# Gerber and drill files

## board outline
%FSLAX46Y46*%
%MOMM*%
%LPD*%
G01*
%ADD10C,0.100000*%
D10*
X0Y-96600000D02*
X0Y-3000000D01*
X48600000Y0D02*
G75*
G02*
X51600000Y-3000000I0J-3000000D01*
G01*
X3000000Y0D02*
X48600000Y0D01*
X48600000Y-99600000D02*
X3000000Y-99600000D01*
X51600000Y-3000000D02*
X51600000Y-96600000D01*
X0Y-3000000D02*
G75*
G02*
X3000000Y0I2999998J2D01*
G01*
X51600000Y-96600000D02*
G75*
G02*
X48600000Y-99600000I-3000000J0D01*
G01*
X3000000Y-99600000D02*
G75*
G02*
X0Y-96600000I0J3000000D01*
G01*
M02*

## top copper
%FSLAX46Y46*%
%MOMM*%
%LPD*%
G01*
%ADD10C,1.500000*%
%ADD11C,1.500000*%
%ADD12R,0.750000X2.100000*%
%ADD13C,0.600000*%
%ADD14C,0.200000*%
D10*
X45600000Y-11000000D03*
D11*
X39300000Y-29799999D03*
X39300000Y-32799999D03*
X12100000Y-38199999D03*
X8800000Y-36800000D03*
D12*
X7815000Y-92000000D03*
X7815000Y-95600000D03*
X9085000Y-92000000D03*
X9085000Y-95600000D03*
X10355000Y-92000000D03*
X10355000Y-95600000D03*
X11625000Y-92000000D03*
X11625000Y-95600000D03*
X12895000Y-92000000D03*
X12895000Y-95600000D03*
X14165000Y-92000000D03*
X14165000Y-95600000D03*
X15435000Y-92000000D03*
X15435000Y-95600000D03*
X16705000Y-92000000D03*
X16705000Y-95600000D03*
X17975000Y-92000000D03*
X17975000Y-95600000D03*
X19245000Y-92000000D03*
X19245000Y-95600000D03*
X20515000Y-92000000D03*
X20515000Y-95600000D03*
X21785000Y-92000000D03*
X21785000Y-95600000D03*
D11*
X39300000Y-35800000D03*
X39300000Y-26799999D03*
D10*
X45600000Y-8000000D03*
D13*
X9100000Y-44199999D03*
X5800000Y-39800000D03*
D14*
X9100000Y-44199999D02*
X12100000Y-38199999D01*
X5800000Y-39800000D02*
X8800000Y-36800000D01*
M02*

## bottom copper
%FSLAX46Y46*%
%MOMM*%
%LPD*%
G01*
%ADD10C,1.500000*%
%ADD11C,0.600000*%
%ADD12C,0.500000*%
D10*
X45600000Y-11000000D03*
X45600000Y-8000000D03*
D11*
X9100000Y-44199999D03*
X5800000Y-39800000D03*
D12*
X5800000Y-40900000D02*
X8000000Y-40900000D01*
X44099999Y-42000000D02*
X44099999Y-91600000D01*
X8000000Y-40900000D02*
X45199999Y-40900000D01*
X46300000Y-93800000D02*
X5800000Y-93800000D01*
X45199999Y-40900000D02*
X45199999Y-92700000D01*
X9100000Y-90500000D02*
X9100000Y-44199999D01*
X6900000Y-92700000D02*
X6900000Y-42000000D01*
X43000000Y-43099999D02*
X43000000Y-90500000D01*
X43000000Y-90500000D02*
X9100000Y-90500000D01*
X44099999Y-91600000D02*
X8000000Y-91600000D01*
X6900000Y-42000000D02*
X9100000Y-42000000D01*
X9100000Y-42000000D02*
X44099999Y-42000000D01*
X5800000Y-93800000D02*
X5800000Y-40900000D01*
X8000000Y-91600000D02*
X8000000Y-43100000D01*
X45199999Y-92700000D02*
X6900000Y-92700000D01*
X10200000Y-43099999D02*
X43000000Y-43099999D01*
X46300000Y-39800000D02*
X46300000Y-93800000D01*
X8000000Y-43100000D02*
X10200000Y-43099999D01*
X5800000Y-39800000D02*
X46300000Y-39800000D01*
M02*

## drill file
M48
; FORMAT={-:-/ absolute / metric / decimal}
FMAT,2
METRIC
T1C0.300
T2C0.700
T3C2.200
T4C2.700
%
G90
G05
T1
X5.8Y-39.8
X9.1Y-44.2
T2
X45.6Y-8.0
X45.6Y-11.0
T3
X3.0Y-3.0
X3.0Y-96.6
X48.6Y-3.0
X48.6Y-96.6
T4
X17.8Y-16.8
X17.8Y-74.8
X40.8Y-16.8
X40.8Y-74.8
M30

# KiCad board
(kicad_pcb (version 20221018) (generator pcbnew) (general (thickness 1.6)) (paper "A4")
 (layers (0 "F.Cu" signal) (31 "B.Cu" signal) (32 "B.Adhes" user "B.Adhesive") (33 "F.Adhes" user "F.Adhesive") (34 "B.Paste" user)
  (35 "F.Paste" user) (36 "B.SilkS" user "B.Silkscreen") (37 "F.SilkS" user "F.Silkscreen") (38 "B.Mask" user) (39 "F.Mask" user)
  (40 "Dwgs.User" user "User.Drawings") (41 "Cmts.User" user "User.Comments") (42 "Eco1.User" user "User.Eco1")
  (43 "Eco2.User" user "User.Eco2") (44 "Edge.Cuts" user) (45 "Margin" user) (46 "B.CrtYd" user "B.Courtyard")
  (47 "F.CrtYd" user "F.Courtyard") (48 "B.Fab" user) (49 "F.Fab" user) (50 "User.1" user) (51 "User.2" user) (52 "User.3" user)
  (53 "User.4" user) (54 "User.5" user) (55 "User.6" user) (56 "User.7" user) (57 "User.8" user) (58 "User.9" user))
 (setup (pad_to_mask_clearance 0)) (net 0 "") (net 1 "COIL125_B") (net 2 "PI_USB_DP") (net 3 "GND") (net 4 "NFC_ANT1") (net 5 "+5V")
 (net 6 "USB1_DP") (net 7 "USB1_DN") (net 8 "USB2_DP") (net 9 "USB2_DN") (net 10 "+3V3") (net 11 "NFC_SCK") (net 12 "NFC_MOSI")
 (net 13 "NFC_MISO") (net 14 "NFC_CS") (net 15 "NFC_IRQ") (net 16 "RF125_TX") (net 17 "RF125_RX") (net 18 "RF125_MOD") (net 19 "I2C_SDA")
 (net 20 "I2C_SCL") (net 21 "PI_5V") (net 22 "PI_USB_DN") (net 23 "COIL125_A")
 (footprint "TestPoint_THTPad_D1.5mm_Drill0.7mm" (layer "F.Cu") (at 45.6 11)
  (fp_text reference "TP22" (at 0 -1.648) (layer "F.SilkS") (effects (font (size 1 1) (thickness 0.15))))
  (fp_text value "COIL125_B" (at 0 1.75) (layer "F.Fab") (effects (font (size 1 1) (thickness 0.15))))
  (pad "1" thru_hole circle (at 0 0) (size 1.5 1.5) (drill 0.7) (layers "*.Cu" "*.Mask") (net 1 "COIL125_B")))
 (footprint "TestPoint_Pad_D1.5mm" (layer "F.Cu") (at 39.3 29.799999)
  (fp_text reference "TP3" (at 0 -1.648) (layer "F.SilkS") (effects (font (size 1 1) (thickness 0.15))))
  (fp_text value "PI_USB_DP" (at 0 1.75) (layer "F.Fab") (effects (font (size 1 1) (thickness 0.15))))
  (pad "1" smd circle (at 0 0) (size 1.5 1.5) (layers "F.Cu" "F.Mask") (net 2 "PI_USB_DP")))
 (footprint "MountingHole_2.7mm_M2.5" (layer "F.Cu") (at 17.8 16.799999)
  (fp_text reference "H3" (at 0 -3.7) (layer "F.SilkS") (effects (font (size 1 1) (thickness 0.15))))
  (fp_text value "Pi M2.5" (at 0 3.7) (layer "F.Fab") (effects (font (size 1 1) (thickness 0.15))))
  (pad "" np_thru_hole circle (at 0 0) (size 2.7 2.7) (drill 2.7) (layers "*.Cu" "*.Mask")))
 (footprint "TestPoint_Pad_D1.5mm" (layer "F.Cu") (at 39.3 32.799999)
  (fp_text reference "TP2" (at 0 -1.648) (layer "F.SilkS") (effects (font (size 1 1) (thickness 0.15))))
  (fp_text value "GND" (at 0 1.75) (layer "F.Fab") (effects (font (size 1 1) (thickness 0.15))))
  (pad "1" smd circle (at 0 0) (size 1.5 1.5) (layers "F.Cu" "F.Mask") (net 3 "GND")))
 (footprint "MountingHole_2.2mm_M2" (layer "F.Cu") (at 48.6 3)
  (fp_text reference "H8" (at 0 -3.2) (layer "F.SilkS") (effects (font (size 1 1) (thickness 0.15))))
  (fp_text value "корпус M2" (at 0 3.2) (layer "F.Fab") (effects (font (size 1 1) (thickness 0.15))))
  (pad "" np_thru_hole circle (at 0 0) (size 2.2 2.2) (drill 2.2) (layers "*.Cu" "*.Mask")))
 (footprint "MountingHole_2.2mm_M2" (layer "F.Cu") (at 3 3)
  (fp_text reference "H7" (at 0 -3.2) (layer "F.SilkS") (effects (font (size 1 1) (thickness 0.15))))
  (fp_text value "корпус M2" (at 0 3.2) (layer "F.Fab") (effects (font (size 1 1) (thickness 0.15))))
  (pad "" np_thru_hole circle (at 0 0) (size 2.2 2.2) (drill 2.2) (layers "*.Cu" "*.Mask")))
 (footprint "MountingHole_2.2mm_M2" (layer "F.Cu") (at 3 96.6)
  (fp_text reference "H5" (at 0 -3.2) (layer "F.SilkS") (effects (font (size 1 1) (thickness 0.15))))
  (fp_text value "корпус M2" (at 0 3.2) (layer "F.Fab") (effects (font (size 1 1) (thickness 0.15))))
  (pad "" np_thru_hole circle (at 0 0) (size 2.2 2.2) (drill 2.2) (layers "*.Cu" "*.Mask")))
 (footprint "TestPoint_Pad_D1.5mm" (layer "F.Cu") (at 12.1 38.199999)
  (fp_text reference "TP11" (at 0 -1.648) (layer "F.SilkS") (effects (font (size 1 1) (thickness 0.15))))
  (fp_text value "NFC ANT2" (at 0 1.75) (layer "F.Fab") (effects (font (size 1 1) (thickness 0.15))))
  (pad "1" smd circle (at 0 0) (size 1.5 1.5) (layers "F.Cu" "F.Mask") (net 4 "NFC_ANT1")))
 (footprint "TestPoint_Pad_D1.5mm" (layer "F.Cu") (at 8.8 36.8)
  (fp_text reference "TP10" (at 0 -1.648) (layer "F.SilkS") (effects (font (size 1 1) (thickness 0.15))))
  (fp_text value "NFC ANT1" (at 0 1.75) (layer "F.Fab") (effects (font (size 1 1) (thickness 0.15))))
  (pad "1" smd circle (at 0 0) (size 1.5 1.5) (layers "F.Cu" "F.Mask") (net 4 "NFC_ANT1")))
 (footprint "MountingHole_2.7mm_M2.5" (layer "F.Cu") (at 40.8 16.799999)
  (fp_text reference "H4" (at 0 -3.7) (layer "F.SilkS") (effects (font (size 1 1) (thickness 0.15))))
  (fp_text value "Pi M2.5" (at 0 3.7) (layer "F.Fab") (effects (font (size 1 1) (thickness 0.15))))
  (pad "" np_thru_hole circle (at 0 0) (size 2.7 2.7) (drill 2.7) (layers "*.Cu" "*.Mask")))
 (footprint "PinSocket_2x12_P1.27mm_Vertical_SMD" (layer "F.Cu") (at 14.8 93.8 90)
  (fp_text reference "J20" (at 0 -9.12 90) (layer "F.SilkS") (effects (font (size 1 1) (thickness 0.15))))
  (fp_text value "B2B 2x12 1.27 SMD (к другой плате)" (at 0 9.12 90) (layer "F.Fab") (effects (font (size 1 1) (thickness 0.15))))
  (pad "1" smd rect (at 1.8 -6.985 90) (size 2.1 0.75) (layers "F.Cu" "F.Paste" "F.Mask") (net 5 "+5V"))
  (pad "2" smd rect (at -1.8 -6.985 90) (size 2.1 0.75) (layers "F.Cu" "F.Paste" "F.Mask") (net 5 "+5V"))
  (pad "3" smd rect (at 1.8 -5.715 90) (size 2.1 0.75) (layers "F.Cu" "F.Paste" "F.Mask") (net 3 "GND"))
  (pad "4" smd rect (at -1.8 -5.715 90) (size 2.1 0.75) (layers "F.Cu" "F.Paste" "F.Mask") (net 3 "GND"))
  (pad "5" smd rect (at 1.8 -4.445 90) (size 2.1 0.75) (layers "F.Cu" "F.Paste" "F.Mask") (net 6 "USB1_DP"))
  (pad "6" smd rect (at -1.8 -4.445 90) (size 2.1 0.75) (layers "F.Cu" "F.Paste" "F.Mask") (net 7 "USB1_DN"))
  (pad "7" smd rect (at 1.8 -3.175 90) (size 2.1 0.75) (layers "F.Cu" "F.Paste" "F.Mask") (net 3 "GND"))
  (pad "8" smd rect (at -1.8 -3.175 90) (size 2.1 0.75) (layers "F.Cu" "F.Paste" "F.Mask") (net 3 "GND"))
  (pad "9" smd rect (at 1.8 -1.905 90) (size 2.1 0.75) (layers "F.Cu" "F.Paste" "F.Mask") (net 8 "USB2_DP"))
  (pad "10" smd rect (at -1.8 -1.905 90) (size 2.1 0.75) (layers "F.Cu" "F.Paste" "F.Mask") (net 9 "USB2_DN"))
  (pad "11" smd rect (at 1.8 -0.635 90) (size 2.1 0.75) (layers "F.Cu" "F.Paste" "F.Mask") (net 3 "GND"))
  (pad "12" smd rect (at -1.8 -0.635 90) (size 2.1 0.75) (layers "F.Cu" "F.Paste" "F.Mask") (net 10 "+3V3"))
  (pad "13" smd rect (at 1.8 0.635 90) (size 2.1 0.75) (layers "F.Cu" "F.Paste" "F.Mask") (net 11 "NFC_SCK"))
  (pad "14" smd rect (at -1.8 0.635 90) (size 2.1 0.75) (layers "F.Cu" "F.Paste" "F.Mask") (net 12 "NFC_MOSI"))
  (pad "15" smd rect (at 1.8 1.905 90) (size 2.1 0.75) (layers "F.Cu" "F.Paste" "F.Mask") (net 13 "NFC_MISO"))
  (pad "16" smd rect (at -1.8 1.905 90) (size 2.1 0.75) (layers "F.Cu" "F.Paste" "F.Mask") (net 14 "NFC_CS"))
  (pad "17" smd rect (at 1.8 3.175 90) (size 2.1 0.75) (layers "F.Cu" "F.Paste" "F.Mask") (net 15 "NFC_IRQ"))
  (pad "18" smd rect (at -1.8 3.175 90) (size 2.1 0.75) (layers "F.Cu" "F.Paste" "F.Mask") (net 3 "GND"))
  (pad "19" smd rect (at 1.8 4.445 90) (size 2.1 0.75) (layers "F.Cu" "F.Paste" "F.Mask") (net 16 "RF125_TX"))
  (pad "20" smd rect (at -1.8 4.445 90) (size 2.1 0.75) (layers "F.Cu" "F.Paste" "F.Mask") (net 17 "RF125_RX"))
  (pad "21" smd rect (at 1.8 5.715 90) (size 2.1 0.75) (layers "F.Cu" "F.Paste" "F.Mask") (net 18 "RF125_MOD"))
  (pad "22" smd rect (at -1.8 5.715 90) (size 2.1 0.75) (layers "F.Cu" "F.Paste" "F.Mask") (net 3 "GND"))
  (pad "23" smd rect (at 1.8 6.985 90) (size 2.1 0.75) (layers "F.Cu" "F.Paste" "F.Mask") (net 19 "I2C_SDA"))
  (pad "24" smd rect (at -1.8 6.985 90) (size 2.1 0.75) (layers "F.Cu" "F.Paste" "F.Mask") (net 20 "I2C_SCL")))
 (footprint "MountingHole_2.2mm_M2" (layer "F.Cu") (at 48.6 96.6)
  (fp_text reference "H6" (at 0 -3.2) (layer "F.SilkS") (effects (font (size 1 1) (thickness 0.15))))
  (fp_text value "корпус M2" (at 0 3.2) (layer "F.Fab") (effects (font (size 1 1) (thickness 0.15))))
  (pad "" np_thru_hole circle (at 0 0) (size 2.2 2.2) (drill 2.2) (layers "*.Cu" "*.Mask")))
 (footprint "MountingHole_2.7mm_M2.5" (layer "F.Cu") (at 40.8 74.8)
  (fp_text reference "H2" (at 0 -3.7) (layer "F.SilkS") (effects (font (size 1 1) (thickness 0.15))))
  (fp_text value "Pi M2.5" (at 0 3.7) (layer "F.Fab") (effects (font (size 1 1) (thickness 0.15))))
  (pad "" np_thru_hole circle (at 0 0) (size 2.7 2.7) (drill 2.7) (layers "*.Cu" "*.Mask")))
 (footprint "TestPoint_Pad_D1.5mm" (layer "F.Cu") (at 39.3 35.8)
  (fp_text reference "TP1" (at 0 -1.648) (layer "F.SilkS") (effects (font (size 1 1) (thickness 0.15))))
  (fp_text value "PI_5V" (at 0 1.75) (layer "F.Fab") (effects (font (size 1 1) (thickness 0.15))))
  (pad "1" smd circle (at 0 0) (size 1.5 1.5) (layers "F.Cu" "F.Mask") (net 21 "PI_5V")))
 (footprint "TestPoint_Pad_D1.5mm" (layer "F.Cu") (at 39.3 26.799999)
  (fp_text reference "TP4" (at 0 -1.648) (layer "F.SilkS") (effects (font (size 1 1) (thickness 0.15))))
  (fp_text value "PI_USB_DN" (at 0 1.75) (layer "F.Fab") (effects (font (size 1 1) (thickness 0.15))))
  (pad "1" smd circle (at 0 0) (size 1.5 1.5) (layers "F.Cu" "F.Mask") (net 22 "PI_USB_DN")))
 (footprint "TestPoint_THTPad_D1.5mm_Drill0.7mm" (layer "F.Cu") (at 45.6 8)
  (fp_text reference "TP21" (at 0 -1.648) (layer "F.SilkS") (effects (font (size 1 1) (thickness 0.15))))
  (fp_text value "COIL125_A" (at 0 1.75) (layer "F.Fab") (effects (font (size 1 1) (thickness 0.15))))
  (pad "1" thru_hole circle (at 0 0) (size 1.5 1.5) (drill 0.7) (layers "*.Cu" "*.Mask") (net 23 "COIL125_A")))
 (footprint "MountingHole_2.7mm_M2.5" (layer "F.Cu") (at 17.8 74.8)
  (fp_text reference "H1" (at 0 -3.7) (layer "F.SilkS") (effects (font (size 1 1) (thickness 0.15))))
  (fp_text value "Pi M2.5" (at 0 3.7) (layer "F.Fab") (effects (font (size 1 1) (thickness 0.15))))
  (pad "" np_thru_hole circle (at 0 0) (size 2.7 2.7) (drill 2.7) (layers "*.Cu" "*.Mask")))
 (gr_line (start 0 96.6) (end 0 3) (stroke (width 0.1) (type default)) (layer "Edge.Cuts"))
 (gr_arc (start 48.6 0) (mid 50.72132 0.878679) (end 51.6 3) (stroke (width 0.1) (type default)) (layer "Edge.Cuts"))
 (gr_line (start 3 0) (end 48.6 0) (stroke (width 0.1) (type default)) (layer "Edge.Cuts"))
 (gr_line (start 48.6 99.6) (end 3 99.6) (stroke (width 0.1) (type default)) (layer "Edge.Cuts"))
 (gr_line (start 51.6 3) (end 51.6 96.6) (stroke (width 0.1) (type default)) (layer "Edge.Cuts"))
 (gr_arc (start 0 3) (mid 0.878679 0.878679) (end 3 0) (stroke (width 0.1) (type default)) (layer "Edge.Cuts"))
 (gr_arc (start 51.6 96.6) (mid 50.72132 98.72132) (end 48.6 99.6) (stroke (width 0.1) (type default)) (layer "Edge.Cuts"))
 (gr_arc (start 3 99.6) (mid 0.878679 98.72132) (end 0 96.6) (stroke (width 0.1) (type default)) (layer "Edge.Cuts"))
 (segment (start 9.1 44.199999) (end 12.1 38.199999) (width 0.2) (layer "F.Cu") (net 4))
 (segment (start 5.8 39.8) (end 8.8 36.8) (width 0.2) (layer "F.Cu") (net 4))
 (via (at 9.1 44.199999) (size 0.6) (drill 0.3) (layers "F.Cu" "B.Cu") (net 4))
 (via (at 5.8 39.8) (size 0.6) (drill 0.3) (layers "F.Cu" "B.Cu") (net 4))
 (segment (start 5.8 40.9) (end 8 40.9) (width 0.5) (layer "B.Cu") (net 4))
 (segment (start 44.099999 42) (end 44.099999 91.6) (width 0.5) (layer "B.Cu") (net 4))
 (segment (start 8 40.9) (end 45.199999 40.9) (width 0.5) (layer "B.Cu") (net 4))
 (segment (start 46.3 93.8) (end 5.8 93.8) (width 0.5) (layer "B.Cu") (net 4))
 (segment (start 45.199999 40.9) (end 45.199999 92.7) (width 0.5) (layer "B.Cu") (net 4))
 (segment (start 9.1 90.5) (end 9.1 44.199999) (width 0.5) (layer "B.Cu") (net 4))
 (segment (start 6.9 92.7) (end 6.9 42) (width 0.5) (layer "B.Cu") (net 4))
 (segment (start 43 43.099999) (end 43 90.5) (width 0.5) (layer "B.Cu") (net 4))
 (segment (start 43 90.5) (end 9.1 90.5) (width 0.5) (layer "B.Cu") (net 4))
 (segment (start 44.099999 91.6) (end 8 91.6) (width 0.5) (layer "B.Cu") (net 4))
 (segment (start 6.9 42) (end 9.1 42) (width 0.5) (layer "B.Cu") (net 4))
 (segment (start 9.1 42) (end 44.099999 42) (width 0.5) (layer "B.Cu") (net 4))
 (segment (start 5.8 93.8) (end 5.8 40.9) (width 0.5) (layer "B.Cu") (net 4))
 (segment (start 8 91.6) (end 8 43.1) (width 0.5) (layer "B.Cu") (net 4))
 (segment (start 45.199999 92.7) (end 6.9 92.7) (width 0.5) (layer "B.Cu") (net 4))
 (segment (start 10.2 43.099999) (end 43 43.099999) (width 0.5) (layer "B.Cu") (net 4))
 (segment (start 46.3 39.8) (end 46.3 93.8) (width 0.5) (layer "B.Cu") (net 4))
 (segment (start 8 43.1) (end 10.2 43.099999) (width 0.5) (layer "B.Cu") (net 4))
 (segment (start 5.8 39.8) (end 46.3 39.8) (width 0.5) (layer "B.Cu") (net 4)))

